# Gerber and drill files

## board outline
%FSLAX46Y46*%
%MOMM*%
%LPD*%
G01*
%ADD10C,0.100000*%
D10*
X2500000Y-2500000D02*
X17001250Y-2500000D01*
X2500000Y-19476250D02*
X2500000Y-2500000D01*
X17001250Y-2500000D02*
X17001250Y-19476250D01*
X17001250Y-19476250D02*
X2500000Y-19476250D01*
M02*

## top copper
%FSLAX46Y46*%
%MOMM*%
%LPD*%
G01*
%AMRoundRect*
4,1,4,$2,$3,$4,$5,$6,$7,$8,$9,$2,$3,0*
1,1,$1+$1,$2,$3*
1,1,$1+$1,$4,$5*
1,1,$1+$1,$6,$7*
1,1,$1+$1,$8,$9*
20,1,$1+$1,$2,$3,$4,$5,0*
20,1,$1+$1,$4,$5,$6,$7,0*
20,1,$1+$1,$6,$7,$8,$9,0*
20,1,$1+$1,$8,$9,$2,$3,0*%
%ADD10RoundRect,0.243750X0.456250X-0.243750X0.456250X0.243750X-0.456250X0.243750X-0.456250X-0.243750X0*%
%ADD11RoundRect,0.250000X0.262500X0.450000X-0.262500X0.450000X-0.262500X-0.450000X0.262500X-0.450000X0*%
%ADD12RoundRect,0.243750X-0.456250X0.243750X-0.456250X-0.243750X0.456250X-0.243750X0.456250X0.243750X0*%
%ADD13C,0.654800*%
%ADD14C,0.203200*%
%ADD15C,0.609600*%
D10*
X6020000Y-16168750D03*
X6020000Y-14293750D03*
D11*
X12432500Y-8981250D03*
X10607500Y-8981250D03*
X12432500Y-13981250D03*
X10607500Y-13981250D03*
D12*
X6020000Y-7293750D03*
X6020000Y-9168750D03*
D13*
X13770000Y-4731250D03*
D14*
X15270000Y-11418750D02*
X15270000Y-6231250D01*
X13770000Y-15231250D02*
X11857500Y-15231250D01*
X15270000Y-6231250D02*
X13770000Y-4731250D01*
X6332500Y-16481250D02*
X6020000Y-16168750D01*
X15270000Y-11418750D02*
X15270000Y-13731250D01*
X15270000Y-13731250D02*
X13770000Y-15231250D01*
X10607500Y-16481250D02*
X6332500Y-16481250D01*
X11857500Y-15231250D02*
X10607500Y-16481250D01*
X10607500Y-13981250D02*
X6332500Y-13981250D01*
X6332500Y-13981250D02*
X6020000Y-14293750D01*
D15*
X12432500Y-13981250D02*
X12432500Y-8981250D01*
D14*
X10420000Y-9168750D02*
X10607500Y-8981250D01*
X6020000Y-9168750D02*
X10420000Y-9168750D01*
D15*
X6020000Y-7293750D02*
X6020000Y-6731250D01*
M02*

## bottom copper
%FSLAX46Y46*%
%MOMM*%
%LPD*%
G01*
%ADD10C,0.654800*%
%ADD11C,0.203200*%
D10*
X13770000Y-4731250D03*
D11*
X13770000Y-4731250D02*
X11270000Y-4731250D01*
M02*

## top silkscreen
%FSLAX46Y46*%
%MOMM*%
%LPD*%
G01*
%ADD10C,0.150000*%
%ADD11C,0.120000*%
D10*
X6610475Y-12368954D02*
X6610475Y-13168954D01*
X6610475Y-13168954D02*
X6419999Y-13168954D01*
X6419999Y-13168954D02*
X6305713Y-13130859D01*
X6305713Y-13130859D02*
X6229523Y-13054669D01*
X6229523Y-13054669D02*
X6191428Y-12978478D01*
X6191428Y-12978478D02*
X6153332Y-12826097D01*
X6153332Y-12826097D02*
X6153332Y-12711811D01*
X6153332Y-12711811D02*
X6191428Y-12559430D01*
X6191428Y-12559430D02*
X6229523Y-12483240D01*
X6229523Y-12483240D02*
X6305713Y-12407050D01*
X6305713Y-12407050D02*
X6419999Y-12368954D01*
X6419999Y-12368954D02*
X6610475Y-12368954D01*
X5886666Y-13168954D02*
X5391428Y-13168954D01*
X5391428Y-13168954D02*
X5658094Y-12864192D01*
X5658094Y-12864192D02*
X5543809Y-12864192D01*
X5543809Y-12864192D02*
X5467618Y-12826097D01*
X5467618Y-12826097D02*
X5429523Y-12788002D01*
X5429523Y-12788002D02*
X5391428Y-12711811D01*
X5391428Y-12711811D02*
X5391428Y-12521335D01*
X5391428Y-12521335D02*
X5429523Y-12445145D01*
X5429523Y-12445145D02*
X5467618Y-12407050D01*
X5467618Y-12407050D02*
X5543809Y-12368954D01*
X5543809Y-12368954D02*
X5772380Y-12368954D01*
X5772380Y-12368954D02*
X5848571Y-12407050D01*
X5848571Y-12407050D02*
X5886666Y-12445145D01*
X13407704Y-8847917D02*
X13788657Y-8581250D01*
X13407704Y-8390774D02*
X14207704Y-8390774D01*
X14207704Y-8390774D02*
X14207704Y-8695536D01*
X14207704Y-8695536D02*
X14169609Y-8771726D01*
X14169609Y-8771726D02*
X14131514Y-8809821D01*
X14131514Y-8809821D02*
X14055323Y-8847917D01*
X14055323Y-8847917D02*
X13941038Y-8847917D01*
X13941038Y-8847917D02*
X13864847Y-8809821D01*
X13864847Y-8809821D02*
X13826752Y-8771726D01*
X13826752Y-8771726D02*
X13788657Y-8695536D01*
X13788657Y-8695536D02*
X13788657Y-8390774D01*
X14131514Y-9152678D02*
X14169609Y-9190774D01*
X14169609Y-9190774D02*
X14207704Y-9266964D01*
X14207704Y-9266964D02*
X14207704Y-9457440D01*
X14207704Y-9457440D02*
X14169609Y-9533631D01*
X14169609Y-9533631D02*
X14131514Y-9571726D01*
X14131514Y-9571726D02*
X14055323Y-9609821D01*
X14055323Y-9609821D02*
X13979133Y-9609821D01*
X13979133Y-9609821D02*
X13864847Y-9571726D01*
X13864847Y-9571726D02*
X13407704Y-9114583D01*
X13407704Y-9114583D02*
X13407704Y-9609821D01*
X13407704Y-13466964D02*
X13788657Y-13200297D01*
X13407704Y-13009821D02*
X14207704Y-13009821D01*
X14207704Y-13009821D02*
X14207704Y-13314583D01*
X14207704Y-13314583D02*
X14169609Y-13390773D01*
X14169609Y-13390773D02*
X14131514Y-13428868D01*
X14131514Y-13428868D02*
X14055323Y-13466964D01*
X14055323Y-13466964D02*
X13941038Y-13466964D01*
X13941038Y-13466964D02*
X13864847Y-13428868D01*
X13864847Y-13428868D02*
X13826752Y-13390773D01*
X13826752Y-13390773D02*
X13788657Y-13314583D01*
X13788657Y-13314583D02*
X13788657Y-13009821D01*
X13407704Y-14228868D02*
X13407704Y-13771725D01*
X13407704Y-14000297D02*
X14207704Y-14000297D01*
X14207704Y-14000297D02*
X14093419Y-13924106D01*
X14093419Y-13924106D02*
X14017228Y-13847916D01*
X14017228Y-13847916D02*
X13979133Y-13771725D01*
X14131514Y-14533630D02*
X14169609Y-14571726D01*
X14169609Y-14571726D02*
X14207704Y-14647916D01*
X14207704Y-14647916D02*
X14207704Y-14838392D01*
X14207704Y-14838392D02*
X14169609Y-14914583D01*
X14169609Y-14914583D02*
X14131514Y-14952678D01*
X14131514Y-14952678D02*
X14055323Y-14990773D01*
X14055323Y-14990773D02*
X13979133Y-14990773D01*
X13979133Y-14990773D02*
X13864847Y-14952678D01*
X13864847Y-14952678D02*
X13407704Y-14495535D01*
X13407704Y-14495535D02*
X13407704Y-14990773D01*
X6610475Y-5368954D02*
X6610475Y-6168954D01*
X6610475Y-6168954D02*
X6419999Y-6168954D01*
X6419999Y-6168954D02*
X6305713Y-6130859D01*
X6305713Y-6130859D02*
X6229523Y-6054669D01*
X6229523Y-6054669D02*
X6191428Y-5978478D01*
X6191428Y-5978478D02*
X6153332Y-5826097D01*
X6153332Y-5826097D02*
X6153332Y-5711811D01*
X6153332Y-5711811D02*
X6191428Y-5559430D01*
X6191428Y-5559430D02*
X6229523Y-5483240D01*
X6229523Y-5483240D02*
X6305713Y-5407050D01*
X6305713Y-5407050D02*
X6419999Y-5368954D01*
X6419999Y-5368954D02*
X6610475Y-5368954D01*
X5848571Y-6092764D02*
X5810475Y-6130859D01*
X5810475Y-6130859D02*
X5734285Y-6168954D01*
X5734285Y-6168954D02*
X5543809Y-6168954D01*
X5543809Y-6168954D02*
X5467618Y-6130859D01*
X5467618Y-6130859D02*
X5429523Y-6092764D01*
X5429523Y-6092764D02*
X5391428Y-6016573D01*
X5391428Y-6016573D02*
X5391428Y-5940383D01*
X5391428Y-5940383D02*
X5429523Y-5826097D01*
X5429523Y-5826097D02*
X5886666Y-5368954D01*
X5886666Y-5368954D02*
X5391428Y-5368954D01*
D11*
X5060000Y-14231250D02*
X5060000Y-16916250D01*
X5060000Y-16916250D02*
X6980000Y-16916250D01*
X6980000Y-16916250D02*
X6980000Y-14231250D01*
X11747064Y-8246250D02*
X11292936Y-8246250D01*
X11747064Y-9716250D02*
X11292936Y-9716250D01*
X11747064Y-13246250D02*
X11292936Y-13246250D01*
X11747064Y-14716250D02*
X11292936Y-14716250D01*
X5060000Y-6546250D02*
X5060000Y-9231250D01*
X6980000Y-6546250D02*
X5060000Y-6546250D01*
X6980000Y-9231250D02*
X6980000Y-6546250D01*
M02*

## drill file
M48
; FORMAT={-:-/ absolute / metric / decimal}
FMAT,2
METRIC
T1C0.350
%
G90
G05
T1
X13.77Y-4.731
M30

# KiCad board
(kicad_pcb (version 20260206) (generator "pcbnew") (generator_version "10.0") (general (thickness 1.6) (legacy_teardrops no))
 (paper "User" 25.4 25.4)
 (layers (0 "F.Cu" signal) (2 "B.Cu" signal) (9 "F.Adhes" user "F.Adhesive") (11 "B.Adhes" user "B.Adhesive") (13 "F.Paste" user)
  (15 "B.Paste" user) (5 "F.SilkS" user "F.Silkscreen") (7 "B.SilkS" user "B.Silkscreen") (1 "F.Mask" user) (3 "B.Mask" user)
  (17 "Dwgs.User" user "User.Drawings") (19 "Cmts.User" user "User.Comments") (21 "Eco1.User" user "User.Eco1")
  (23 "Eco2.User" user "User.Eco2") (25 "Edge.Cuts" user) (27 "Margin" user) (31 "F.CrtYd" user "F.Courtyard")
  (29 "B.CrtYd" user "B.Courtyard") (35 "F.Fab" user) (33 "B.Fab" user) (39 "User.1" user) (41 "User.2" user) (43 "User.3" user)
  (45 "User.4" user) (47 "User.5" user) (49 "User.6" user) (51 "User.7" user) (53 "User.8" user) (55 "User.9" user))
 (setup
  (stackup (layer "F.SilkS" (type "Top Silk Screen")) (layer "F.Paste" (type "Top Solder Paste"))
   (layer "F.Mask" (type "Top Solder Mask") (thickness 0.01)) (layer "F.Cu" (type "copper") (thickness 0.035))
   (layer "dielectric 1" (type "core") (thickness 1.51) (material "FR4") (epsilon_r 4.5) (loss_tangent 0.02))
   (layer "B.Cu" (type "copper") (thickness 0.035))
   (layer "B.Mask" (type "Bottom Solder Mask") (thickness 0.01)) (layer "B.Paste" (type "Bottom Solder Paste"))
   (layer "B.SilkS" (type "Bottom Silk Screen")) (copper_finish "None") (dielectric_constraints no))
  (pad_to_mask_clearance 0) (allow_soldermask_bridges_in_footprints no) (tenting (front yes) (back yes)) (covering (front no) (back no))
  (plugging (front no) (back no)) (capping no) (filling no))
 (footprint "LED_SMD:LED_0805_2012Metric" (layer "F.Cu") (at 6.02 15.23125 90)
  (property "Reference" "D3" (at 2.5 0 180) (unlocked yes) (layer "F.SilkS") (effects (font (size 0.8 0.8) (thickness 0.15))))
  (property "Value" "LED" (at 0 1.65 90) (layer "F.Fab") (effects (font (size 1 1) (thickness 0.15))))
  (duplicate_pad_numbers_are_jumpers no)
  (fp_line (start 1 -0.96) (end -1.685 -0.96) (stroke (width 0.12) (type solid)) (layer "F.SilkS"))
  (fp_line (start -1.685 -0.96) (end -1.685 0.96) (stroke (width 0.12) (type solid)) (layer "F.SilkS"))
  (fp_line (start -1.685 0.96) (end 1 0.96) (stroke (width 0.12) (type solid)) (layer "F.SilkS"))
  (pad "1" smd roundrect (at -0.9375 0 90) (size 0.975 1.4) (layers "F.Cu" "F.Mask" "F.Paste") (roundrect_rratio 0.25) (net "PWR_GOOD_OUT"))
  (pad "2" smd roundrect (at 0.9375 0 90) (size 0.975 1.4) (layers "F.Cu" "F.Mask" "F.Paste") (roundrect_rratio 0.25) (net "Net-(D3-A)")))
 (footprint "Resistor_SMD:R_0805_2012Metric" (layer "F.Cu") (at 11.52 8.98125 180)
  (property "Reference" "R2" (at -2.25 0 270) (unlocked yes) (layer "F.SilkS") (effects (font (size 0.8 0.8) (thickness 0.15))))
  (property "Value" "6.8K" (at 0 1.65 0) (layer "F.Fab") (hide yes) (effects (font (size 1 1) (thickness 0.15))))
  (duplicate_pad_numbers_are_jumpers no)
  (fp_line (start -0.227064 0.735) (end 0.227064 0.735) (stroke (width 0.12) (type solid)) (layer "F.SilkS"))
  (fp_line (start -0.227064 -0.735) (end 0.227064 -0.735) (stroke (width 0.12) (type solid)) (layer "F.SilkS"))
  (pad "1" smd roundrect (at -0.9125 0 180) (size 1.025 1.4) (layers "F.Cu" "F.Mask" "F.Paste") (roundrect_rratio 0.243902439) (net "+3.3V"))
  (pad "2" smd roundrect (at 0.9125 0 180) (size 1.025 1.4) (layers "F.Cu" "F.Mask" "F.Paste") (roundrect_rratio 0.243902439)
   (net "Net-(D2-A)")))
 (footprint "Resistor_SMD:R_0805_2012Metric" (layer "F.Cu") (at 11.52 13.98125 180)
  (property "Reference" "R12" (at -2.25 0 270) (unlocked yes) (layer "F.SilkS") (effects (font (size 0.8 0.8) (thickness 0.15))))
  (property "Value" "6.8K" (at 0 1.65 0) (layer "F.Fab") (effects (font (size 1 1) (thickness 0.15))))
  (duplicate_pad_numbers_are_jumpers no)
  (fp_line (start -0.227064 0.735) (end 0.227064 0.735) (stroke (width 0.12) (type solid)) (layer "F.SilkS"))
  (fp_line (start -0.227064 -0.735) (end 0.227064 -0.735) (stroke (width 0.12) (type solid)) (layer "F.SilkS"))
  (pad "1" smd roundrect (at -0.9125 0 180) (size 1.025 1.4) (layers "F.Cu" "F.Mask" "F.Paste") (roundrect_rratio 0.243902) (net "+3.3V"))
  (pad "2" smd roundrect (at 0.9125 0 180) (size 1.025 1.4) (layers "F.Cu" "F.Mask" "F.Paste") (roundrect_rratio 0.243902)
   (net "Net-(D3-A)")))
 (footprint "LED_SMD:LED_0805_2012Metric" (layer "F.Cu") (at 6.02 8.23125 -90)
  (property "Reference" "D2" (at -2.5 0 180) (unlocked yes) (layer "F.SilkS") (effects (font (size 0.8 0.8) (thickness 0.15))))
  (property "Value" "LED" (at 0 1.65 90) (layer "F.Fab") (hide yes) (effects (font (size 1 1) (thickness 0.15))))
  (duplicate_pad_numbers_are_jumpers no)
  (fp_line (start -1.685 0.96) (end 1 0.96) (stroke (width 0.12) (type solid)) (layer "F.SilkS"))
  (fp_line (start -1.685 -0.96) (end -1.685 0.96) (stroke (width 0.12) (type solid)) (layer "F.SilkS"))
  (fp_line (start 1 -0.96) (end -1.685 -0.96) (stroke (width 0.12) (type solid)) (layer "F.SilkS"))
  (pad "1" smd roundrect (at -0.9375 0 270) (size 0.975 1.4) (layers "F.Cu" "F.Mask" "F.Paste") (roundrect_rratio 0.25) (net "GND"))
  (pad "2" smd roundrect (at 0.9375 0 270) (size 0.975 1.4) (layers "F.Cu" "F.Mask" "F.Paste") (roundrect_rratio 0.25) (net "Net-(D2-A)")))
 (gr_line (start 2.5 2.5) (end 17.00125 2.5) (stroke (width 0.1) (type default)) (layer "Edge.Cuts"))
 (gr_line (start 2.5 19.47625) (end 2.5 2.5) (stroke (width 0.1) (type default)) (layer "Edge.Cuts"))
 (gr_line (start 17.00125 2.5) (end 17.00125 19.47625) (stroke (width 0.1) (type default)) (layer "Edge.Cuts"))
 (gr_line (start 17.00125 19.47625) (end 2.5 19.47625) (stroke (width 0.1) (type default)) (layer "Edge.Cuts"))
 (segment (start 15.27 11.41875) (end 15.27 6.23125) (width 0.2032) (layer "F.Cu") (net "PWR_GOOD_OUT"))
 (segment (start 13.77 15.23125) (end 11.8575 15.23125) (width 0.2032) (layer "F.Cu") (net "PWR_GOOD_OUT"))
 (segment (start 15.27 6.23125) (end 13.77 4.73125) (width 0.2032) (layer "F.Cu") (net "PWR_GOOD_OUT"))
 (segment (start 6.3325 16.48125) (end 6.02 16.16875) (width 0.2032) (layer "F.Cu") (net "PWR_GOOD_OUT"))
 (segment (start 15.27 11.41875) (end 15.27 13.73125) (width 0.2032) (layer "F.Cu") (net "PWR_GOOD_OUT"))
 (segment (start 15.27 13.73125) (end 13.77 15.23125) (width 0.2032) (layer "F.Cu") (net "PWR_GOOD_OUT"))
 (segment (start 10.6075 16.48125) (end 6.3325 16.48125) (width 0.2032) (layer "F.Cu") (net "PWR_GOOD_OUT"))
 (segment (start 11.8575 15.23125) (end 10.6075 16.48125) (width 0.2032) (layer "F.Cu") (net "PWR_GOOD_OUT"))
 (via (at 13.77 4.73125) (size 0.6548) (drill 0.35) (layers "F.Cu" "B.Cu") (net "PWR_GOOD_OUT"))
 (segment (start 13.77 4.73125) (end 11.27 4.73125) (width 0.2032) (layer "B.Cu") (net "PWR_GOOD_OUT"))
 (segment (start 10.6075 13.98125) (end 6.3325 13.98125) (width 0.2032) (layer "F.Cu") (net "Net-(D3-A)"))
 (segment (start 6.3325 13.98125) (end 6.02 14.29375) (width 0.2032) (layer "F.Cu") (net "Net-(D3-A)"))
 (segment (start 12.4325 13.98125) (end 12.4325 8.98125) (width 0.6096) (layer "F.Cu") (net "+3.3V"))
 (segment (start 10.42 9.16875) (end 10.6075 8.98125) (width 0.2032) (layer "F.Cu") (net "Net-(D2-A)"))
 (segment (start 6.02 9.16875) (end 10.42 9.16875) (width 0.2032) (layer "F.Cu") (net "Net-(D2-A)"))
 (segment (start 6.02 7.29375) (end 6.02 6.73125) (width 0.6096) (layer "F.Cu") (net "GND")))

